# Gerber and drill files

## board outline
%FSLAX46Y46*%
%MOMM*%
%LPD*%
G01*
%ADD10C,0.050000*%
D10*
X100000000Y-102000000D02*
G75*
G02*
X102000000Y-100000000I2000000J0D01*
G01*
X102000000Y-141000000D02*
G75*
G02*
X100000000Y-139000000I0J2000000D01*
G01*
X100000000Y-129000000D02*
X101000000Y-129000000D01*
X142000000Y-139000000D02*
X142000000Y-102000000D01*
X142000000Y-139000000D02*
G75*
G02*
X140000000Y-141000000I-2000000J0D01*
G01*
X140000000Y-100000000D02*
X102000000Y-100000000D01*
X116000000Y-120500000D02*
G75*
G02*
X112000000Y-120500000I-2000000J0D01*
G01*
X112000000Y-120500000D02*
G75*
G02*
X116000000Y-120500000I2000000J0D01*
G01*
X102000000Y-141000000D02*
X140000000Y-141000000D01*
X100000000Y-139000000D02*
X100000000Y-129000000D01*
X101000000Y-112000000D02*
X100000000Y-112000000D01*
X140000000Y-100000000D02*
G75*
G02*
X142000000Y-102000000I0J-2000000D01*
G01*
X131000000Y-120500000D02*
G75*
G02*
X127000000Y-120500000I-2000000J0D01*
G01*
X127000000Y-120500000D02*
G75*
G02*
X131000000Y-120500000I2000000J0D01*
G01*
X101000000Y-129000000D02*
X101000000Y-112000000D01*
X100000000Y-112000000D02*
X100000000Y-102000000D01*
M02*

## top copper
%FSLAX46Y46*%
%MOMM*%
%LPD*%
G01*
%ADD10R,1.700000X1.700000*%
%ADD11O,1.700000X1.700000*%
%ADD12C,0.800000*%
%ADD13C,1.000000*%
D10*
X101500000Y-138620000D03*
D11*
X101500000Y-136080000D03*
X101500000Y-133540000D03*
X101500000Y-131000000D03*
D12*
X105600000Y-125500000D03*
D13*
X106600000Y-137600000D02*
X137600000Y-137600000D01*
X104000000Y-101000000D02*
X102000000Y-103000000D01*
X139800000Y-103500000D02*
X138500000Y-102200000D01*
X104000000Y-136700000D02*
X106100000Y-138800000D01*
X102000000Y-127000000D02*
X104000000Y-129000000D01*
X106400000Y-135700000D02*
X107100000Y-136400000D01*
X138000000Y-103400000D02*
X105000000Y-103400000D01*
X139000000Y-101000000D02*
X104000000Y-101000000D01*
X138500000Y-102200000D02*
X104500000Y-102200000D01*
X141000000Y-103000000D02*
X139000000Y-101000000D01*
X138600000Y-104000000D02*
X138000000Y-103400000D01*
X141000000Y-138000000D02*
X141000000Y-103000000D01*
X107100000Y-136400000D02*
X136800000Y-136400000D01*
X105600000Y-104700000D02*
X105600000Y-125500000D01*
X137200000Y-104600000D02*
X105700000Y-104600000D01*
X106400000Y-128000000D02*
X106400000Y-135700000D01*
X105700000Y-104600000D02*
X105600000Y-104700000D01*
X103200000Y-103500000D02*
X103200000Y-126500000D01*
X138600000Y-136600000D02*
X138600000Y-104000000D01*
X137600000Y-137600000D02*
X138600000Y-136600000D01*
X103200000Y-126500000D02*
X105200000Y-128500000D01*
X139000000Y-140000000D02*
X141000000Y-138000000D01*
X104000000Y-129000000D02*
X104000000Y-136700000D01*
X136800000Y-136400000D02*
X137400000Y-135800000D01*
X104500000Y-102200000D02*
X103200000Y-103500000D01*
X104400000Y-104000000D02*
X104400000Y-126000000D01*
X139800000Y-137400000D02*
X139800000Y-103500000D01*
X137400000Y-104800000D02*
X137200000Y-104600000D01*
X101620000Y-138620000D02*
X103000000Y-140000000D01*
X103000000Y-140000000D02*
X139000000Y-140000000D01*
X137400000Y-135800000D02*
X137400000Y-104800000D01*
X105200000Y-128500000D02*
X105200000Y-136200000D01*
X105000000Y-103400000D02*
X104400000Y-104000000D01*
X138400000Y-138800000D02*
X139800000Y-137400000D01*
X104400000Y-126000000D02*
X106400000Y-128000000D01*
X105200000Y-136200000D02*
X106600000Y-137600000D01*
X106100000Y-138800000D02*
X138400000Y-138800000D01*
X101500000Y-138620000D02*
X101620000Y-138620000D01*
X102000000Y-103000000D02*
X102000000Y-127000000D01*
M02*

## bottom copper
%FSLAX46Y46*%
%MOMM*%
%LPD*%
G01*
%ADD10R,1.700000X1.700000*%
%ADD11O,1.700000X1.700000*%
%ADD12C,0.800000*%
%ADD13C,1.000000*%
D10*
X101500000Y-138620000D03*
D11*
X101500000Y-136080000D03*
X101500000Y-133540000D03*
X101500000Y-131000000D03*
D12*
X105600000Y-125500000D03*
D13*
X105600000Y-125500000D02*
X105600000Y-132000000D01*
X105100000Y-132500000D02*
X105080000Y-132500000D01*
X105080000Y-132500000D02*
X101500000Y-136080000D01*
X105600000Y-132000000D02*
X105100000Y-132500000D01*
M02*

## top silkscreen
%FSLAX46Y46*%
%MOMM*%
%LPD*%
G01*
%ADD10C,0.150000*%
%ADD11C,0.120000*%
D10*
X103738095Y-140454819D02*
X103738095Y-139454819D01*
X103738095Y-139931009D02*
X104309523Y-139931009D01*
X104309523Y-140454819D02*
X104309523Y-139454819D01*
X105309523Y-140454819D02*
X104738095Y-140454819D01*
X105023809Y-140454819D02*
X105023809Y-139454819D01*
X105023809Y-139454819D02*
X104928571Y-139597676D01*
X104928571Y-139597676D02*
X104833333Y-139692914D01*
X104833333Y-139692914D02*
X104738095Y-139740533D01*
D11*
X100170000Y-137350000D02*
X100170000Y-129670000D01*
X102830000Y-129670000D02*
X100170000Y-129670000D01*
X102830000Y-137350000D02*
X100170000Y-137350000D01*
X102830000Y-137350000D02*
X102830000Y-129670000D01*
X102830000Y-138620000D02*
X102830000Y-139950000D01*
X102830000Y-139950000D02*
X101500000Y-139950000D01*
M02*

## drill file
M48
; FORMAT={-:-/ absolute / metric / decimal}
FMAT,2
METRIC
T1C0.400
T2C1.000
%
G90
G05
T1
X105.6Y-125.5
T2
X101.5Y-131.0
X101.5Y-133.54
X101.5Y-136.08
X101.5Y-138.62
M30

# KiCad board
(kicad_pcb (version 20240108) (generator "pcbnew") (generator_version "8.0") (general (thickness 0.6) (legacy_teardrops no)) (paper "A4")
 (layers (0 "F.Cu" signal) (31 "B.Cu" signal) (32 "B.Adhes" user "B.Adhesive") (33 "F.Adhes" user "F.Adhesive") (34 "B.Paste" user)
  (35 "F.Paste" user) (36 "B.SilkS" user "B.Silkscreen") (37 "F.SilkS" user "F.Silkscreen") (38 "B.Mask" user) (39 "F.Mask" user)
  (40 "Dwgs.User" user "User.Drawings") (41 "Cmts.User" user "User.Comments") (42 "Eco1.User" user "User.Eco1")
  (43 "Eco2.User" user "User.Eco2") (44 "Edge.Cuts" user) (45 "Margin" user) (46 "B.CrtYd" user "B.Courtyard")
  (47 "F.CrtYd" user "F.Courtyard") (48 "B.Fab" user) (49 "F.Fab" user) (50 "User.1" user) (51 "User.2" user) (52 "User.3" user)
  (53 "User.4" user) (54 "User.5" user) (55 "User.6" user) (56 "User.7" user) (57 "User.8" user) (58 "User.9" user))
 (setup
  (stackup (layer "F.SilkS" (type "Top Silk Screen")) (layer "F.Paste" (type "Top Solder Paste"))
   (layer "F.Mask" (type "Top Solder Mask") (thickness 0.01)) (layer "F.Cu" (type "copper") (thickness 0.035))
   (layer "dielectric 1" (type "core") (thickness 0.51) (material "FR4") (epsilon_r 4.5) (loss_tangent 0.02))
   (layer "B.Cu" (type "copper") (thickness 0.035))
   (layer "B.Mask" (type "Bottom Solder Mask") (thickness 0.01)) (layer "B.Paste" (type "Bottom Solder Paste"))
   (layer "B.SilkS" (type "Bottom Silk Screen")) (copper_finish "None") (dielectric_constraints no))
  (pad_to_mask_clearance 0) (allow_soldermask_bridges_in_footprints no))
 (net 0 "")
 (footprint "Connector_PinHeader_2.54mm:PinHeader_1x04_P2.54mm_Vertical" (layer "F.Cu") (at 101.5 138.62 180)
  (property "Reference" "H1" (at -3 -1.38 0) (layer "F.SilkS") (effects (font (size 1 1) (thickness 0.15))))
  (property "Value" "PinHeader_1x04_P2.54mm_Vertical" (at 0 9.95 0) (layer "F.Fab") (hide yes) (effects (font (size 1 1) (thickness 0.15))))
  (fp_line (start 1.33 1.27) (end 1.33 8.95) (stroke (width 0.12) (type solid)) (layer "F.SilkS"))
  (fp_line (start -1.33 8.95) (end 1.33 8.95) (stroke (width 0.12) (type solid)) (layer "F.SilkS"))
  (fp_line (start -1.33 1.27) (end 1.33 1.27) (stroke (width 0.12) (type solid)) (layer "F.SilkS"))
  (fp_line (start -1.33 1.27) (end -1.33 8.95) (stroke (width 0.12) (type solid)) (layer "F.SilkS"))
  (fp_line (start -1.33 0) (end -1.33 -1.33) (stroke (width 0.12) (type solid)) (layer "F.SilkS"))
  (fp_line (start -1.33 -1.33) (end 0 -1.33) (stroke (width 0.12) (type solid)) (layer "F.SilkS"))
  (pad "1" thru_hole rect (at 0 0 180) (size 1.7 1.7) (drill 1) (layers "*.Cu" "*.Mask") (remove_unused_layers no))
  (pad "2" thru_hole oval (at 0 2.54 180) (size 1.7 1.7) (drill 1) (layers "*.Cu" "*.Mask") (remove_unused_layers no))
  (pad "3" thru_hole oval (at 0 5.08 180) (size 1.7 1.7) (drill 1) (layers "*.Cu" "*.Mask") (remove_unused_layers no))
  (pad "4" thru_hole oval (at 0 7.62 180) (size 1.7 1.7) (drill 1) (layers "*.Cu" "*.Mask") (remove_unused_layers no)))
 (gr_arc (start 100 102) (mid 100.585786 100.585786) (end 102 100) (stroke (width 0.05) (type default)) (layer "Edge.Cuts"))
 (gr_arc (start 102 141) (mid 100.585786 140.414214) (end 100 139) (stroke (width 0.05) (type default)) (layer "Edge.Cuts"))
 (gr_line (start 100 129) (end 101 129) (stroke (width 0.05) (type default)) (layer "Edge.Cuts"))
 (gr_line (start 142 139) (end 142 102) (stroke (width 0.05) (type default)) (layer "Edge.Cuts"))
 (gr_arc (start 142 139) (mid 141.414214 140.414214) (end 140 141) (stroke (width 0.05) (type default)) (layer "Edge.Cuts"))
 (gr_line (start 140 100) (end 102 100) (stroke (width 0.05) (type default)) (layer "Edge.Cuts"))
 (gr_circle (center 114 120.5) (end 116 120.5) (stroke (width 0.05) (type default)) (fill none) (layer "Edge.Cuts"))
 (gr_line (start 102 141) (end 140 141) (stroke (width 0.05) (type default)) (layer "Edge.Cuts"))
 (gr_line (start 100 139) (end 100 129) (stroke (width 0.05) (type default)) (layer "Edge.Cuts"))
 (gr_line (start 101 112) (end 100 112) (stroke (width 0.05) (type default)) (layer "Edge.Cuts"))
 (gr_arc (start 140 100) (mid 141.414214 100.585786) (end 142 102) (stroke (width 0.05) (type default)) (layer "Edge.Cuts"))
 (gr_circle (center 129 120.5) (end 131 120.5) (stroke (width 0.05) (type default)) (fill none) (layer "Edge.Cuts"))
 (gr_line (start 101 129) (end 101 112) (stroke (width 0.05) (type default)) (layer "Edge.Cuts"))
 (gr_line (start 100 112) (end 100 102) (stroke (width 0.05) (type default)) (layer "Edge.Cuts"))
 (segment (start 106.6 137.6) (end 137.6 137.6) (width 1) (layer "F.Cu") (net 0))
 (segment (start 104 101) (end 102 103) (width 1) (layer "F.Cu") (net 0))
 (segment (start 139.8 103.5) (end 138.5 102.2) (width 1) (layer "F.Cu") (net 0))
 (segment (start 104 136.7) (end 106.1 138.8) (width 1) (layer "F.Cu") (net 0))
 (segment (start 102 127) (end 104 129) (width 1) (layer "F.Cu") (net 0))
 (segment (start 106.4 135.7) (end 107.1 136.4) (width 1) (layer "F.Cu") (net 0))
 (segment (start 138 103.4) (end 105 103.4) (width 1) (layer "F.Cu") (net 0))
 (segment (start 139 101) (end 104 101) (width 1) (layer "F.Cu") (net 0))
 (segment (start 138.5 102.2) (end 104.5 102.2) (width 1) (layer "F.Cu") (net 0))
 (segment (start 141 103) (end 139 101) (width 1) (layer "F.Cu") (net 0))
 (segment (start 138.6 104) (end 138 103.4) (width 1) (layer "F.Cu") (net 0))
 (segment (start 141 138) (end 141 103) (width 1) (layer "F.Cu") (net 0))
 (segment (start 107.1 136.4) (end 136.8 136.4) (width 1) (layer "F.Cu") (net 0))
 (segment (start 105.6 104.7) (end 105.6 125.5) (width 1) (layer "F.Cu") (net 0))
 (segment (start 137.2 104.6) (end 105.7 104.6) (width 1) (layer "F.Cu") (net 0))
 (segment (start 106.4 128) (end 106.4 135.7) (width 1) (layer "F.Cu") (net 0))
 (segment (start 105.7 104.6) (end 105.6 104.7) (width 1) (layer "F.Cu") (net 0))
 (segment (start 103.2 103.5) (end 103.2 126.5) (width 1) (layer "F.Cu") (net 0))
 (segment (start 138.6 136.6) (end 138.6 104) (width 1) (layer "F.Cu") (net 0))
 (segment (start 137.6 137.6) (end 138.6 136.6) (width 1) (layer "F.Cu") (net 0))
 (segment (start 103.2 126.5) (end 105.2 128.5) (width 1) (layer "F.Cu") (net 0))
 (segment (start 139 140) (end 141 138) (width 1) (layer "F.Cu") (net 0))
 (segment (start 104 129) (end 104 136.7) (width 1) (layer "F.Cu") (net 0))
 (segment (start 136.8 136.4) (end 137.4 135.8) (width 1) (layer "F.Cu") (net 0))
 (segment (start 104.5 102.2) (end 103.2 103.5) (width 1) (layer "F.Cu") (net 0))
 (segment (start 104.4 104) (end 104.4 126) (width 1) (layer "F.Cu") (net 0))
 (segment (start 139.8 137.4) (end 139.8 103.5) (width 1) (layer "F.Cu") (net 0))
 (segment (start 137.4 104.8) (end 137.2 104.6) (width 1) (layer "F.Cu") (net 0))
 (segment (start 101.62 138.62) (end 103 140) (width 1) (layer "F.Cu") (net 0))
 (segment (start 103 140) (end 139 140) (width 1) (layer "F.Cu") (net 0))
 (segment (start 137.4 135.8) (end 137.4 104.8) (width 1) (layer "F.Cu") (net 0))
 (segment (start 105.2 128.5) (end 105.2 136.2) (width 1) (layer "F.Cu") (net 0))
 (segment (start 105 103.4) (end 104.4 104) (width 1) (layer "F.Cu") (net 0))
 (segment (start 138.4 138.8) (end 139.8 137.4) (width 1) (layer "F.Cu") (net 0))
 (segment (start 104.4 126) (end 106.4 128) (width 1) (layer "F.Cu") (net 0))
 (segment (start 105.2 136.2) (end 106.6 137.6) (width 1) (layer "F.Cu") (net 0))
 (segment (start 106.1 138.8) (end 138.4 138.8) (width 1) (layer "F.Cu") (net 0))
 (segment (start 101.5 138.62) (end 101.62 138.62) (width 1) (layer "F.Cu") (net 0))
 (segment (start 102 103) (end 102 127) (width 1) (layer "F.Cu") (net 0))
 (via (at 105.6 125.5) (size 0.8) (drill 0.4) (layers "F.Cu" "B.Cu") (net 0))
 (segment (start 105.6 125.5) (end 105.6 132) (width 1) (layer "B.Cu") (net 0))
 (segment (start 105.1 132.5) (end 105.08 132.5) (width 1) (layer "B.Cu") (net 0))
 (segment (start 105.08 132.5) (end 101.5 136.08) (width 1) (layer "B.Cu") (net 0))
 (segment (start 105.6 132) (end 105.1 132.5) (width 1) (layer "B.Cu") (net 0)))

